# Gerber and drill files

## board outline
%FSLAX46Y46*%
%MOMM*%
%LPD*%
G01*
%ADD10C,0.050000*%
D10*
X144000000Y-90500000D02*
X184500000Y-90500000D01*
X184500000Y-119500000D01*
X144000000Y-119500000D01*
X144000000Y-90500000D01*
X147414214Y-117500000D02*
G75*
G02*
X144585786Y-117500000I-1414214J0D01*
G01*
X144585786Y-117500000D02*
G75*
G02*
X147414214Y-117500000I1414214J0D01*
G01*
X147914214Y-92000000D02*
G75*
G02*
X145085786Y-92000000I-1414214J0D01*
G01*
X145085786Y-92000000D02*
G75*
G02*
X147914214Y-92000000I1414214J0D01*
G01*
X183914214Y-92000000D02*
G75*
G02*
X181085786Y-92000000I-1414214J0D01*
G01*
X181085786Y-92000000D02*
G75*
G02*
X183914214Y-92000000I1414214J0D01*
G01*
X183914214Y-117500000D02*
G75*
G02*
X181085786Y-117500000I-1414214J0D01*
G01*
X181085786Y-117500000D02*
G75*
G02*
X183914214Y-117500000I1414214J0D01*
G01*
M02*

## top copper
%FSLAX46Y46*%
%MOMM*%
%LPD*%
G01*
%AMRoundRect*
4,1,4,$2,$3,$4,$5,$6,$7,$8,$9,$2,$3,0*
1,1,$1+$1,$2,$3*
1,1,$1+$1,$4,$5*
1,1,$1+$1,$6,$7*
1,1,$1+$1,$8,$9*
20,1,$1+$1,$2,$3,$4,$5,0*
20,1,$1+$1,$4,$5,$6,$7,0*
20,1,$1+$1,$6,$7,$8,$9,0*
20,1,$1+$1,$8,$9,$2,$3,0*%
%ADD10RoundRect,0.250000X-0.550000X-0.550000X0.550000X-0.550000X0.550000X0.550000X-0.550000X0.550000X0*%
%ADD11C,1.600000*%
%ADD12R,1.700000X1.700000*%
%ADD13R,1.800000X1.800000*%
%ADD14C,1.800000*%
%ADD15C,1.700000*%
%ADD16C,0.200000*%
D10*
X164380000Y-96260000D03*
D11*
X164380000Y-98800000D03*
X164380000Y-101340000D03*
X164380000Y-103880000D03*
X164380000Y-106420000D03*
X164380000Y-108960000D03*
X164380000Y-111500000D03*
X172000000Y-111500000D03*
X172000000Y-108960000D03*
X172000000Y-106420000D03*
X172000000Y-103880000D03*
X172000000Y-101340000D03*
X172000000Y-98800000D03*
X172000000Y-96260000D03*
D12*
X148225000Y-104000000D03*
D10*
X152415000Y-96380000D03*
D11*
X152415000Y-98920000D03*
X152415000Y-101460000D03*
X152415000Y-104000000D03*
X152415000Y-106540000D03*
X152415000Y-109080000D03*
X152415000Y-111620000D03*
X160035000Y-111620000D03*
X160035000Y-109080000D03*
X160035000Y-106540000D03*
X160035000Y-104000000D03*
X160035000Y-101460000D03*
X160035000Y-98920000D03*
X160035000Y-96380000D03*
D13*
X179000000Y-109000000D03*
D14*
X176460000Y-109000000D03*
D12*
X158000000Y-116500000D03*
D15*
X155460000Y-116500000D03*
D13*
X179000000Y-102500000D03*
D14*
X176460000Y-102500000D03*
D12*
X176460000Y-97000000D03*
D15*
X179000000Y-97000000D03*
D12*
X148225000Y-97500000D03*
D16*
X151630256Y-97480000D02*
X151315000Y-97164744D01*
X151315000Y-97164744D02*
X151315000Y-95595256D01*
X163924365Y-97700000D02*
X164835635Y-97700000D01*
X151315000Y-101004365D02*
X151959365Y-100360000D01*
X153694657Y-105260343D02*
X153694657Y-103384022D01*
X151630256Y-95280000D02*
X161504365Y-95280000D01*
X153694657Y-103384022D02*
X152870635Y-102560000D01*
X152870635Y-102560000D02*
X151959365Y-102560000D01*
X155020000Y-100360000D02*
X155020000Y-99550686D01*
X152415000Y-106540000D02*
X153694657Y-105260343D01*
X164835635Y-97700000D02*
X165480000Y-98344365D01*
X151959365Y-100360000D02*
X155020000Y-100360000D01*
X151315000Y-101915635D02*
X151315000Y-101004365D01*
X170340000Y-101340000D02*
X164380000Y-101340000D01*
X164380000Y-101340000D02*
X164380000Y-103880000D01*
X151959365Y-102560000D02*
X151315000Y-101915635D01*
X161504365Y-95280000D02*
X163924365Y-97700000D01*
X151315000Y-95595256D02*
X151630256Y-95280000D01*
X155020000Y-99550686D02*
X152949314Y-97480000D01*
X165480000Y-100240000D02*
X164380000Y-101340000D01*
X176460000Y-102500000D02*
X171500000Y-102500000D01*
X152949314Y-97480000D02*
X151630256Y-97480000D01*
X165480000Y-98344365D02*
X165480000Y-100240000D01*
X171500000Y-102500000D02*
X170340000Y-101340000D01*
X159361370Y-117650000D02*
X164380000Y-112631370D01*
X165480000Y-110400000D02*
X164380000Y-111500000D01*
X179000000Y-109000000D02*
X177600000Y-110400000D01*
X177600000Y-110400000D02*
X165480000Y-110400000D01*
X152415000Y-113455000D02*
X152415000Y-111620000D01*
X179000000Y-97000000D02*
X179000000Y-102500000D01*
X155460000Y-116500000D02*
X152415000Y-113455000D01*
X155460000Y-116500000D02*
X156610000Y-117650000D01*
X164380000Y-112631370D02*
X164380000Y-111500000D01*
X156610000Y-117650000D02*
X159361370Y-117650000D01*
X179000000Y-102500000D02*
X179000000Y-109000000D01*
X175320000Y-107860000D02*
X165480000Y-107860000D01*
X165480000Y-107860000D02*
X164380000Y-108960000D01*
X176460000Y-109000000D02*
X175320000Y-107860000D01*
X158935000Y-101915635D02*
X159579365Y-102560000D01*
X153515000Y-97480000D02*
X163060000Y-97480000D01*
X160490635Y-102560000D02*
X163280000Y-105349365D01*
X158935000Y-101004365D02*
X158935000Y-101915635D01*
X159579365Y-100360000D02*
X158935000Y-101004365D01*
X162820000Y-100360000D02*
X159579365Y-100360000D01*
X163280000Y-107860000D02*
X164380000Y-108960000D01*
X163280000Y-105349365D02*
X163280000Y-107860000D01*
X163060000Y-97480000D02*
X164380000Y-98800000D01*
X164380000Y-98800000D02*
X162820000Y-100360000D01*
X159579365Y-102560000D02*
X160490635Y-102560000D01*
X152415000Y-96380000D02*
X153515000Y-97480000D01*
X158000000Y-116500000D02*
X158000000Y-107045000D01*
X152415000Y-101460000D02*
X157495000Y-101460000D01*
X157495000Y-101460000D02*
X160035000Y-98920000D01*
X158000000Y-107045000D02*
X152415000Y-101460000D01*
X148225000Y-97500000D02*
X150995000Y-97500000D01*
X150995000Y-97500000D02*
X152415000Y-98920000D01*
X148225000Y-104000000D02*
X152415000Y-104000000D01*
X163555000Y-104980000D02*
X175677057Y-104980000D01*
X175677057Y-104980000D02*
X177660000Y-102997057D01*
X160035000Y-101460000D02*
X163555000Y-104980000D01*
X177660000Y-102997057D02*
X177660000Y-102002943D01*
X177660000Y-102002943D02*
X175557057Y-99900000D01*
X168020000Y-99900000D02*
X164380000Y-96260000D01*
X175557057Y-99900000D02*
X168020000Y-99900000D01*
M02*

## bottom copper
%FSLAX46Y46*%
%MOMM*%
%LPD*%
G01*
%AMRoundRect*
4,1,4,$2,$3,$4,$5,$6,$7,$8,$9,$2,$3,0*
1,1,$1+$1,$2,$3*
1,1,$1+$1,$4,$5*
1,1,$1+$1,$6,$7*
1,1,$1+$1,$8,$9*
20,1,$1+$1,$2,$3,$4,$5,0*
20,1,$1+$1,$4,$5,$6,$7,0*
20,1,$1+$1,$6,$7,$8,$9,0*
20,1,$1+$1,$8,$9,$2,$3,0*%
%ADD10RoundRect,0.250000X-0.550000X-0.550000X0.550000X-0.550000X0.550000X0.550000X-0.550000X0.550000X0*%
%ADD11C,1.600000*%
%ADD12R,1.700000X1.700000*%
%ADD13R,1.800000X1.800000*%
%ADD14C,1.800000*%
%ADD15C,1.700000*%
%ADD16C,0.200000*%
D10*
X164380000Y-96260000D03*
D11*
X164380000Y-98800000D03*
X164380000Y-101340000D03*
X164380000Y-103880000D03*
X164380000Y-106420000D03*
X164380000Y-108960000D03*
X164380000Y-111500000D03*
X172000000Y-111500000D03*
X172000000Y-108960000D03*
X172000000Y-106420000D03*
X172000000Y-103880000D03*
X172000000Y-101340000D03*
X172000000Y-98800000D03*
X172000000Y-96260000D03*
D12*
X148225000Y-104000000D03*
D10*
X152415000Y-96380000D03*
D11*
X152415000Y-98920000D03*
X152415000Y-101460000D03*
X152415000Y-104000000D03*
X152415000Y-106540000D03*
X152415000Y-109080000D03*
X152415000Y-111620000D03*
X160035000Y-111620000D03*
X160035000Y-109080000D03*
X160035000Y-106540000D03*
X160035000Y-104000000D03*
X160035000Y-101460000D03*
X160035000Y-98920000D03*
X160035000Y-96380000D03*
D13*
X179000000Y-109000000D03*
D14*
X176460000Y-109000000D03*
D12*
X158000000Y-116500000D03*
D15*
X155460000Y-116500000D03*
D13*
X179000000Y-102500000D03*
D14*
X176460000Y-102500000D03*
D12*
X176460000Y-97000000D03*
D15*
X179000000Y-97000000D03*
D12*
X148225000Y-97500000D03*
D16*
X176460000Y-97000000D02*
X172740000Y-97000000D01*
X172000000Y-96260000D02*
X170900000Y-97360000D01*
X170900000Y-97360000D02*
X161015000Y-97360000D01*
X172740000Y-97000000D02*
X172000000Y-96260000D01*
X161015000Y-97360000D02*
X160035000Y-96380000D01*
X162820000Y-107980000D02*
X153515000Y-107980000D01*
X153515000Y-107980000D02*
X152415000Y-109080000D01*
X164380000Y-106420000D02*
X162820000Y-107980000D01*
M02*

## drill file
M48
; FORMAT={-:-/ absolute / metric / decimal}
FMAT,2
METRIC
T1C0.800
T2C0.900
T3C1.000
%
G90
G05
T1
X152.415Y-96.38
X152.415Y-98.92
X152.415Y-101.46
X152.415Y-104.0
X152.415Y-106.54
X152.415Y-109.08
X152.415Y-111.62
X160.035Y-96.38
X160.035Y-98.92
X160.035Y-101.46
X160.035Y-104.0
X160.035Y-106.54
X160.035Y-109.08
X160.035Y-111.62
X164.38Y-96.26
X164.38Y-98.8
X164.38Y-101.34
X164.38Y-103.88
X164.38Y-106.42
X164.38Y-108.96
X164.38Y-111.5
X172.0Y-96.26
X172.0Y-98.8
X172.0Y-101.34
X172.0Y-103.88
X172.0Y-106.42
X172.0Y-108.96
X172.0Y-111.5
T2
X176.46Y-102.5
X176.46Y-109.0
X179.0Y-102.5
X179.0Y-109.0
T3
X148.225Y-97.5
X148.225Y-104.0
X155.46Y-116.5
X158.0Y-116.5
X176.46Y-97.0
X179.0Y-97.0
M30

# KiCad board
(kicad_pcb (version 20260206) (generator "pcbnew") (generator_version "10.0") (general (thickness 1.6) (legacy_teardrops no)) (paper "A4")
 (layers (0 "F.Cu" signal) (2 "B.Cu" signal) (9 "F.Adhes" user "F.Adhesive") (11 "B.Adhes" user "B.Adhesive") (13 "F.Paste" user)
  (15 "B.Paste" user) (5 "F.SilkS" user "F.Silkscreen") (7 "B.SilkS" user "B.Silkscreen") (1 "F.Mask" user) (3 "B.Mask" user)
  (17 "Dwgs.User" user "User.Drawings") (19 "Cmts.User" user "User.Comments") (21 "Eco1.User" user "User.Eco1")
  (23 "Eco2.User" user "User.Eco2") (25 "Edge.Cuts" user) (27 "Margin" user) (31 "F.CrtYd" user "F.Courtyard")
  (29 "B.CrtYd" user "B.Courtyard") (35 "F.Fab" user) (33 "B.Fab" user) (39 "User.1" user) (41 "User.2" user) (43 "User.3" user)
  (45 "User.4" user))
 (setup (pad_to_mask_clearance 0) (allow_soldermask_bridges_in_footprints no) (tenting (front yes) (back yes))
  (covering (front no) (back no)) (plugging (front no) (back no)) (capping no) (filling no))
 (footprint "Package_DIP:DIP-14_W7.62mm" (layer "F.Cu") (at 164.38 96.26)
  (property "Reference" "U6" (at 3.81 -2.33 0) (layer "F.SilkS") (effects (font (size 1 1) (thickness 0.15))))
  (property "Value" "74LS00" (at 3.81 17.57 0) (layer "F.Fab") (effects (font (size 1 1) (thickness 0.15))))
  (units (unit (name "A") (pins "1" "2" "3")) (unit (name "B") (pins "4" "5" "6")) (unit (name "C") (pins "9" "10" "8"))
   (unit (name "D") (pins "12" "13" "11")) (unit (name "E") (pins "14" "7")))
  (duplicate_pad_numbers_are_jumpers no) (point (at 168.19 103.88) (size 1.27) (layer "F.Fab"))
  (pad "1" thru_hole roundrect (at 0 0) (size 1.6 1.6) (drill 0.8) (layers "*.Cu" "*.Mask") (remove_unused_layers no)
   (roundrect_rratio 0.15625) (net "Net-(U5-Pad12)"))
  (pad "2" thru_hole circle (at 0 2.54) (size 1.6 1.6) (drill 0.8) (layers "*.Cu" "*.Mask") (remove_unused_layers no) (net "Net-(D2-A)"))
  (pad "3" thru_hole circle (at 0 5.08) (size 1.6 1.6) (drill 0.8) (layers "*.Cu" "*.Mask") (remove_unused_layers no) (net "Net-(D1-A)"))
  (pad "4" thru_hole circle (at 0 7.62) (size 1.6 1.6) (drill 0.8) (layers "*.Cu" "*.Mask") (remove_unused_layers no) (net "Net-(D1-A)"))
  (pad "5" thru_hole circle (at 0 10.16) (size 1.6 1.6) (drill 0.8) (layers "*.Cu" "*.Mask") (remove_unused_layers no) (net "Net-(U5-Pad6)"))
  (pad "6" thru_hole circle (at 0 12.7) (size 1.6 1.6) (drill 0.8) (layers "*.Cu" "*.Mask") (remove_unused_layers no) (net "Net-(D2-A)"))
  (pad "7" thru_hole circle (at 0 15.24) (size 1.6 1.6) (drill 0.8) (layers "*.Cu" "*.Mask") (remove_unused_layers no) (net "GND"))
  (pad "8" thru_hole circle (at 7.62 15.24) (size 1.6 1.6) (drill 0.8) (layers "*.Cu" "*.Mask") (remove_unused_layers no))
  (pad "9" thru_hole circle (at 7.62 12.7) (size 1.6 1.6) (drill 0.8) (layers "*.Cu" "*.Mask") (remove_unused_layers no))
  (pad "10" thru_hole circle (at 7.62 10.16) (size 1.6 1.6) (drill 0.8) (layers "*.Cu" "*.Mask") (remove_unused_layers no))
  (pad "11" thru_hole circle (at 7.62 7.62) (size 1.6 1.6) (drill 0.8) (layers "*.Cu" "*.Mask") (remove_unused_layers no))
  (pad "12" thru_hole circle (at 7.62 5.08) (size 1.6 1.6) (drill 0.8) (layers "*.Cu" "*.Mask") (remove_unused_layers no))
  (pad "13" thru_hole circle (at 7.62 2.54) (size 1.6 1.6) (drill 0.8) (layers "*.Cu" "*.Mask") (remove_unused_layers no))
  (pad "14" thru_hole circle (at 7.62 0) (size 1.6 1.6) (drill 0.8) (layers "*.Cu" "*.Mask") (remove_unused_layers no) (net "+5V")))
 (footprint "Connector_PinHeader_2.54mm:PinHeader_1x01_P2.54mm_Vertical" (layer "F.Cu") (at 148.225 104)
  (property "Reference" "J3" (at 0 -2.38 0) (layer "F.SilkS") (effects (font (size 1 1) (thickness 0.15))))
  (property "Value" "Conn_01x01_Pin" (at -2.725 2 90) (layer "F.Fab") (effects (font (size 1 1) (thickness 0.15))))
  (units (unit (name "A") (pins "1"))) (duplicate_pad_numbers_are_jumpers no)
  (pad "1" thru_hole rect (at 0 0) (size 1.7 1.7) (drill 1) (layers "*.Cu" "*.Mask") (remove_unused_layers no) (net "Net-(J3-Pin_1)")))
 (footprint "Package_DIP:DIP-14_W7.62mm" (layer "F.Cu") (at 152.415 96.38)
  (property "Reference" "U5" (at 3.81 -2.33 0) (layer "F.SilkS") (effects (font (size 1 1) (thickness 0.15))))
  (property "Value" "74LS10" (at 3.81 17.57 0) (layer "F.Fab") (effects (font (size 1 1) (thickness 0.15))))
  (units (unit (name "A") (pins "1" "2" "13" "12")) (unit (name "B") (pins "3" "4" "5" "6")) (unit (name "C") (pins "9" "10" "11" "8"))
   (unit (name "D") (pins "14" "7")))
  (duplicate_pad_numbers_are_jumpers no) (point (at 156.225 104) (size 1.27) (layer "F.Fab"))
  (pad "1" thru_hole roundrect (at 0 0) (size 1.6 1.6) (drill 0.8) (layers "*.Cu" "*.Mask") (remove_unused_layers no)
   (roundrect_rratio 0.15625) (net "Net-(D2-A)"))
  (pad "2" thru_hole circle (at 0 2.54) (size 1.6 1.6) (drill 0.8) (layers "*.Cu" "*.Mask") (remove_unused_layers no) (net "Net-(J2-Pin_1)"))
  (pad "3" thru_hole circle (at 0 5.08) (size 1.6 1.6) (drill 0.8) (layers "*.Cu" "*.Mask") (remove_unused_layers no) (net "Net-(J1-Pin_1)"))
  (pad "4" thru_hole circle (at 0 7.62) (size 1.6 1.6) (drill 0.8) (layers "*.Cu" "*.Mask") (remove_unused_layers no) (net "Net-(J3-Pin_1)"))
  (pad "5" thru_hole circle (at 0 10.16) (size 1.6 1.6) (drill 0.8) (layers "*.Cu" "*.Mask") (remove_unused_layers no) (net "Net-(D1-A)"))
  (pad "6" thru_hole circle (at 0 12.7) (size 1.6 1.6) (drill 0.8) (layers "*.Cu" "*.Mask") (remove_unused_layers no) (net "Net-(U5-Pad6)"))
  (pad "7" thru_hole circle (at 0 15.24) (size 1.6 1.6) (drill 0.8) (layers "*.Cu" "*.Mask") (remove_unused_layers no) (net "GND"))
  (pad "8" thru_hole circle (at 7.62 15.24) (size 1.6 1.6) (drill 0.8) (layers "*.Cu" "*.Mask") (remove_unused_layers no))
  (pad "9" thru_hole circle (at 7.62 12.7) (size 1.6 1.6) (drill 0.8) (layers "*.Cu" "*.Mask") (remove_unused_layers no))
  (pad "10" thru_hole circle (at 7.62 10.16) (size 1.6 1.6) (drill 0.8) (layers "*.Cu" "*.Mask") (remove_unused_layers no))
  (pad "11" thru_hole circle (at 7.62 7.62) (size 1.6 1.6) (drill 0.8) (layers "*.Cu" "*.Mask") (remove_unused_layers no))
  (pad "12" thru_hole circle (at 7.62 5.08) (size 1.6 1.6) (drill 0.8) (layers "*.Cu" "*.Mask") (remove_unused_layers no)
   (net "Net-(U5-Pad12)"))
  (pad "13" thru_hole circle (at 7.62 2.54) (size 1.6 1.6) (drill 0.8) (layers "*.Cu" "*.Mask") (remove_unused_layers no)
   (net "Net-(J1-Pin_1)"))
  (pad "14" thru_hole circle (at 7.62 0) (size 1.6 1.6) (drill 0.8) (layers "*.Cu" "*.Mask") (remove_unused_layers no) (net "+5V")))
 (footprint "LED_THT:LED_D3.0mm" (layer "F.Cu") (at 179 109 180)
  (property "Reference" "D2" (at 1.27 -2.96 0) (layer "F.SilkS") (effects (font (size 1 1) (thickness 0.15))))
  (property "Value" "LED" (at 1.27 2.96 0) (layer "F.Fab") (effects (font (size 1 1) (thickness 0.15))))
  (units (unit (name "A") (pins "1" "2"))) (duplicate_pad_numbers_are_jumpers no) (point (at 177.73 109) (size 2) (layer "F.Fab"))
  (pad "1" thru_hole rect (at 0 0 180) (size 1.8 1.8) (drill 0.9) (layers "*.Cu" "*.Mask") (remove_unused_layers no) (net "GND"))
  (pad "2" thru_hole circle (at 2.54 0 180) (size 1.8 1.8) (drill 0.9) (layers "*.Cu" "*.Mask") (remove_unused_layers no) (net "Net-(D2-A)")))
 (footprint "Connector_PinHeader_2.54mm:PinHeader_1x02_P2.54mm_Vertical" (layer "F.Cu") (at 158 116.5 -90)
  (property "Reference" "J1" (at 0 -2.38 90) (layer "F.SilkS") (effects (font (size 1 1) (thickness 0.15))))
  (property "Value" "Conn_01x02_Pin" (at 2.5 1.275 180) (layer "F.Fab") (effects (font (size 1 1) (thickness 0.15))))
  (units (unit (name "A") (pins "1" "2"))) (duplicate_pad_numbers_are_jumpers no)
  (pad "1" thru_hole rect (at 0 0 270) (size 1.7 1.7) (drill 1) (layers "*.Cu" "*.Mask") (remove_unused_layers no) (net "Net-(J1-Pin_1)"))
  (pad "2" thru_hole circle (at 0 2.54 270) (size 1.7 1.7) (drill 1) (layers "*.Cu" "*.Mask") (remove_unused_layers no) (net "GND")))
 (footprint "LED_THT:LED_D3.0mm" (layer "F.Cu") (at 179 102.5 180)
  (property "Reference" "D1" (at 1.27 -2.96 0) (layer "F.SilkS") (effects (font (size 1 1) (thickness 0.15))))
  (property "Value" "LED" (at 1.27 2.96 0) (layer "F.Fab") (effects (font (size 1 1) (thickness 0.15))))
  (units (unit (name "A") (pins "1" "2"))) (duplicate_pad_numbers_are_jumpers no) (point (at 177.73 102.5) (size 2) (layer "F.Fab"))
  (pad "1" thru_hole rect (at 0 0 180) (size 1.8 1.8) (drill 0.9) (layers "*.Cu" "*.Mask") (remove_unused_layers no) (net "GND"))
  (pad "2" thru_hole circle (at 2.54 0 180) (size 1.8 1.8) (drill 0.9) (layers "*.Cu" "*.Mask") (remove_unused_layers no) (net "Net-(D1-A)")))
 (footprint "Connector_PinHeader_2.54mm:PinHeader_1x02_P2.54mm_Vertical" (layer "F.Cu") (at 176.46 97 90)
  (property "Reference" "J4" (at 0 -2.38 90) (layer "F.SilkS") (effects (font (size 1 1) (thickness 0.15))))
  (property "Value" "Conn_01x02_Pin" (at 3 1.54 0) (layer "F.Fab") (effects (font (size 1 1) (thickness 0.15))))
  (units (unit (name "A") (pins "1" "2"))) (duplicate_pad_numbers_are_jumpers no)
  (pad "1" thru_hole rect (at 0 0 90) (size 1.7 1.7) (drill 1) (layers "*.Cu" "*.Mask") (remove_unused_layers no) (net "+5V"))
  (pad "2" thru_hole circle (at 0 2.54 90) (size 1.7 1.7) (drill 1) (layers "*.Cu" "*.Mask") (remove_unused_layers no) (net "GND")))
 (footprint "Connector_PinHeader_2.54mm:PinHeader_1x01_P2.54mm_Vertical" (layer "F.Cu") (at 148.225 97.5)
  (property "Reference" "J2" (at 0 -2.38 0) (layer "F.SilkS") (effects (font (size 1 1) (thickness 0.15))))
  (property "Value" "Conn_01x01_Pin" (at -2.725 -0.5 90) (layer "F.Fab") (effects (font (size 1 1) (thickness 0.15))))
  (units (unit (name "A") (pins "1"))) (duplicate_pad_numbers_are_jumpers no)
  (pad "1" thru_hole rect (at 0 0) (size 1.7 1.7) (drill 1) (layers "*.Cu" "*.Mask") (remove_unused_layers no) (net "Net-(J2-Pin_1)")))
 (gr_rect (start 144 90.5) (end 184.5 119.5) (stroke (width 0.05) (type default)) (fill no) (layer "Edge.Cuts"))
 (gr_circle (center 146 117.5) (end 147 118.5) (stroke (width 0.05) (type default)) (fill no) (layer "Edge.Cuts"))
 (gr_circle (center 146.5 92) (end 147.5 93) (stroke (width 0.05) (type default)) (fill no) (layer "Edge.Cuts"))
 (gr_circle (center 182.5 92) (end 183.5 93) (stroke (width 0.05) (type default)) (fill no) (layer "Edge.Cuts"))
 (gr_circle (center 182.5 117.5) (end 183.5 118.5) (stroke (width 0.05) (type default)) (fill no) (layer "Edge.Cuts"))
 (segment (start 151.630256 97.48) (end 151.315 97.164744) (width 0.2) (layer "F.Cu") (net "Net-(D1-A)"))
 (segment (start 151.315 97.164744) (end 151.315 95.595256) (width 0.2) (layer "F.Cu") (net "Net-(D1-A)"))
 (segment (start 163.924365 97.7) (end 164.835635 97.7) (width 0.2) (layer "F.Cu") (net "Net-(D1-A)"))
 (segment (start 151.315 101.004365) (end 151.959365 100.36) (width 0.2) (layer "F.Cu") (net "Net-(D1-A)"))
 (segment (start 153.694657 105.260343) (end 153.694657 103.384022) (width 0.2) (layer "F.Cu") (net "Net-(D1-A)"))
 (segment (start 151.630256 95.28) (end 161.504365 95.28) (width 0.2) (layer "F.Cu") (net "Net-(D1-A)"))
 (segment (start 153.694657 103.384022) (end 152.870635 102.56) (width 0.2) (layer "F.Cu") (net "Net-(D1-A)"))
 (segment (start 152.870635 102.56) (end 151.959365 102.56) (width 0.2) (layer "F.Cu") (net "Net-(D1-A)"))
 (segment (start 155.02 100.36) (end 155.02 99.550686) (width 0.2) (layer "F.Cu") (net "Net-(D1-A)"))
 (segment (start 152.415 106.54) (end 153.694657 105.260343) (width 0.2) (layer "F.Cu") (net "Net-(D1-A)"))
 (segment (start 164.835635 97.7) (end 165.48 98.344365) (width 0.2) (layer "F.Cu") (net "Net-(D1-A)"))
 (segment (start 151.959365 100.36) (end 155.02 100.36) (width 0.2) (layer "F.Cu") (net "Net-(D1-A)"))
 (segment (start 151.315 101.915635) (end 151.315 101.004365) (width 0.2) (layer "F.Cu") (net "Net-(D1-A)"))
 (segment (start 170.34 101.34) (end 164.38 101.34) (width 0.2) (layer "F.Cu") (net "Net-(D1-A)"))
 (segment (start 164.38 101.34) (end 164.38 103.88) (width 0.2) (layer "F.Cu") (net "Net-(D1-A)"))
 (segment (start 151.959365 102.56) (end 151.315 101.915635) (width 0.2) (layer "F.Cu") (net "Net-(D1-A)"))
 (segment (start 161.504365 95.28) (end 163.924365 97.7) (width 0.2) (layer "F.Cu") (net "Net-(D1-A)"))
 (segment (start 151.315 95.595256) (end 151.630256 95.28) (width 0.2) (layer "F.Cu") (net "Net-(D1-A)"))
 (segment (start 155.02 99.550686) (end 152.949314 97.48) (width 0.2) (layer "F.Cu") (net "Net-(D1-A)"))
 (segment (start 165.48 100.24) (end 164.38 101.34) (width 0.2) (layer "F.Cu") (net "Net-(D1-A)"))
 (segment (start 176.46 102.5) (end 171.5 102.5) (width 0.2) (layer "F.Cu") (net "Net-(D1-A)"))
 (segment (start 152.949314 97.48) (end 151.630256 97.48) (width 0.2) (layer "F.Cu") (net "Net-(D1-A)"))
 (segment (start 165.48 98.344365) (end 165.48 100.24) (width 0.2) (layer "F.Cu") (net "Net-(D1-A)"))
 (segment (start 171.5 102.5) (end 170.34 101.34) (width 0.2) (layer "F.Cu") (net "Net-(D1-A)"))
 (segment (start 159.36137 117.65) (end 164.38 112.63137) (width 0.2) (layer "F.Cu") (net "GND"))
 (segment (start 165.48 110.4) (end 164.38 111.5) (width 0.2) (layer "F.Cu") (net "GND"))
 (segment (start 179 109) (end 177.6 110.4) (width 0.2) (layer "F.Cu") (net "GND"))
 (segment (start 177.6 110.4) (end 165.48 110.4) (width 0.2) (layer "F.Cu") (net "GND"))
 (segment (start 152.415 113.455) (end 152.415 111.62) (width 0.2) (layer "F.Cu") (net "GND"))
 (segment (start 179 97) (end 179 102.5) (width 0.2) (layer "F.Cu") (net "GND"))
 (segment (start 155.46 116.5) (end 152.415 113.455) (width 0.2) (layer "F.Cu") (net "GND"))
 (segment (start 155.46 116.5) (end 156.61 117.65) (width 0.2) (layer "F.Cu") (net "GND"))
 (segment (start 164.38 112.63137) (end 164.38 111.5) (width 0.2) (layer "F.Cu") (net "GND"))
 (segment (start 156.61 117.65) (end 159.36137 117.65) (width 0.2) (layer "F.Cu") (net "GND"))
 (segment (start 179 102.5) (end 179 109) (width 0.2) (layer "F.Cu") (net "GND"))
 (segment (start 175.32 107.86) (end 165.48 107.86) (width 0.2) (layer "F.Cu") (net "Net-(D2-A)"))
 (segment (start 165.48 107.86) (end 164.38 108.96) (width 0.2) (layer "F.Cu") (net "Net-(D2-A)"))
 (segment (start 176.46 109) (end 175.32 107.86) (width 0.2) (layer "F.Cu") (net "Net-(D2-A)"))
 (segment (start 158.935 101.915635) (end 159.579365 102.56) (width 0.2) (layer "F.Cu") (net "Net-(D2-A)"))
 (segment (start 153.515 97.48) (end 163.06 97.48) (width 0.2) (layer "F.Cu") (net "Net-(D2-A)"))
 (segment (start 160.490635 102.56) (end 163.28 105.349365) (width 0.2) (layer "F.Cu") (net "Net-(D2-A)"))
 (segment (start 158.935 101.004365) (end 158.935 101.915635) (width 0.2) (layer "F.Cu") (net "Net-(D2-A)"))
 (segment (start 159.579365 100.36) (end 158.935 101.004365) (width 0.2) (layer "F.Cu") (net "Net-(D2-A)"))
 (segment (start 162.82 100.36) (end 159.579365 100.36) (width 0.2) (layer "F.Cu") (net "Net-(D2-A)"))
 (segment (start 163.28 107.86) (end 164.38 108.96) (width 0.2) (layer "F.Cu") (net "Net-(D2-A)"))
 (segment (start 163.28 105.349365) (end 163.28 107.86) (width 0.2) (layer "F.Cu") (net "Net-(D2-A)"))
 (segment (start 163.06 97.48) (end 164.38 98.8) (width 0.2) (layer "F.Cu") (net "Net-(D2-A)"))
 (segment (start 164.38 98.8) (end 162.82 100.36) (width 0.2) (layer "F.Cu") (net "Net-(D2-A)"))
 (segment (start 159.579365 102.56) (end 160.490635 102.56) (width 0.2) (layer "F.Cu") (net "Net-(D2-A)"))
 (segment (start 152.415 96.38) (end 153.515 97.48) (width 0.2) (layer "F.Cu") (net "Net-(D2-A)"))
 (segment (start 158 116.5) (end 158 107.045) (width 0.2) (layer "F.Cu") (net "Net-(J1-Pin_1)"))
 (segment (start 152.415 101.46) (end 157.495 101.46) (width 0.2) (layer "F.Cu") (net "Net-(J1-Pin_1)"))
 (segment (start 157.495 101.46) (end 160.035 98.92) (width 0.2) (layer "F.Cu") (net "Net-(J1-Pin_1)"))
 (segment (start 158 107.045) (end 152.415 101.46) (width 0.2) (layer "F.Cu") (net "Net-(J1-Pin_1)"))
 (segment (start 148.225 97.5) (end 150.995 97.5) (width 0.2) (layer "F.Cu") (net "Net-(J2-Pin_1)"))
 (segment (start 150.995 97.5) (end 152.415 98.92) (width 0.2) (layer "F.Cu") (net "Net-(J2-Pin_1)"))
 (segment (start 148.225 104) (end 152.415 104) (width 0.2) (layer "F.Cu") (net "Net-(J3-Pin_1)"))
 (segment (start 176.46 97) (end 172.74 97) (width 0.2) (layer "B.Cu") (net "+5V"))
 (segment (start 172 96.26) (end 170.9 97.36) (width 0.2) (layer "B.Cu") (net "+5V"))
 (segment (start 170.9 97.36) (end 161.015 97.36) (width 0.2) (layer "B.Cu") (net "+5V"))
 (segment (start 172.74 97) (end 172 96.26) (width 0.2) (layer "B.Cu") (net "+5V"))
 (segment (start 161.015 97.36) (end 160.035 96.38) (width 0.2) (layer "B.Cu") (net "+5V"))
 (segment (start 163.555 104.98) (end 175.677057 104.98) (width 0.2) (layer "F.Cu") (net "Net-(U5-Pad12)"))
 (segment (start 175.677057 104.98) (end 177.66 102.997057) (width 0.2) (layer "F.Cu") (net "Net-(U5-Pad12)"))
 (segment (start 160.035 101.46) (end 163.555 104.98) (width 0.2) (layer "F.Cu") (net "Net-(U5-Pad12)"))
 (segment (start 177.66 102.997057) (end 177.66 102.002943) (width 0.2) (layer "F.Cu") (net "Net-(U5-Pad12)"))
 (segment (start 177.66 102.002943) (end 175.557057 99.9) (width 0.2) (layer "F.Cu") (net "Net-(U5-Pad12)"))
 (segment (start 168.02 99.9) (end 164.38 96.26) (width 0.2) (layer "F.Cu") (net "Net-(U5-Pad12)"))
 (segment (start 175.557057 99.9) (end 168.02 99.9) (width 0.2) (layer "F.Cu") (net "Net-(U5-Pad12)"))
 (segment (start 162.82 107.98) (end 153.515 107.98) (width 0.2) (layer "B.Cu") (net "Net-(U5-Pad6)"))
 (segment (start 153.515 107.98) (end 152.415 109.08) (width 0.2) (layer "B.Cu") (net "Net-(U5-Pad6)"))
 (segment (start 164.38 106.42) (end 162.82 107.98) (width 0.2) (layer "B.Cu") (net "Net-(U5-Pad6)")))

